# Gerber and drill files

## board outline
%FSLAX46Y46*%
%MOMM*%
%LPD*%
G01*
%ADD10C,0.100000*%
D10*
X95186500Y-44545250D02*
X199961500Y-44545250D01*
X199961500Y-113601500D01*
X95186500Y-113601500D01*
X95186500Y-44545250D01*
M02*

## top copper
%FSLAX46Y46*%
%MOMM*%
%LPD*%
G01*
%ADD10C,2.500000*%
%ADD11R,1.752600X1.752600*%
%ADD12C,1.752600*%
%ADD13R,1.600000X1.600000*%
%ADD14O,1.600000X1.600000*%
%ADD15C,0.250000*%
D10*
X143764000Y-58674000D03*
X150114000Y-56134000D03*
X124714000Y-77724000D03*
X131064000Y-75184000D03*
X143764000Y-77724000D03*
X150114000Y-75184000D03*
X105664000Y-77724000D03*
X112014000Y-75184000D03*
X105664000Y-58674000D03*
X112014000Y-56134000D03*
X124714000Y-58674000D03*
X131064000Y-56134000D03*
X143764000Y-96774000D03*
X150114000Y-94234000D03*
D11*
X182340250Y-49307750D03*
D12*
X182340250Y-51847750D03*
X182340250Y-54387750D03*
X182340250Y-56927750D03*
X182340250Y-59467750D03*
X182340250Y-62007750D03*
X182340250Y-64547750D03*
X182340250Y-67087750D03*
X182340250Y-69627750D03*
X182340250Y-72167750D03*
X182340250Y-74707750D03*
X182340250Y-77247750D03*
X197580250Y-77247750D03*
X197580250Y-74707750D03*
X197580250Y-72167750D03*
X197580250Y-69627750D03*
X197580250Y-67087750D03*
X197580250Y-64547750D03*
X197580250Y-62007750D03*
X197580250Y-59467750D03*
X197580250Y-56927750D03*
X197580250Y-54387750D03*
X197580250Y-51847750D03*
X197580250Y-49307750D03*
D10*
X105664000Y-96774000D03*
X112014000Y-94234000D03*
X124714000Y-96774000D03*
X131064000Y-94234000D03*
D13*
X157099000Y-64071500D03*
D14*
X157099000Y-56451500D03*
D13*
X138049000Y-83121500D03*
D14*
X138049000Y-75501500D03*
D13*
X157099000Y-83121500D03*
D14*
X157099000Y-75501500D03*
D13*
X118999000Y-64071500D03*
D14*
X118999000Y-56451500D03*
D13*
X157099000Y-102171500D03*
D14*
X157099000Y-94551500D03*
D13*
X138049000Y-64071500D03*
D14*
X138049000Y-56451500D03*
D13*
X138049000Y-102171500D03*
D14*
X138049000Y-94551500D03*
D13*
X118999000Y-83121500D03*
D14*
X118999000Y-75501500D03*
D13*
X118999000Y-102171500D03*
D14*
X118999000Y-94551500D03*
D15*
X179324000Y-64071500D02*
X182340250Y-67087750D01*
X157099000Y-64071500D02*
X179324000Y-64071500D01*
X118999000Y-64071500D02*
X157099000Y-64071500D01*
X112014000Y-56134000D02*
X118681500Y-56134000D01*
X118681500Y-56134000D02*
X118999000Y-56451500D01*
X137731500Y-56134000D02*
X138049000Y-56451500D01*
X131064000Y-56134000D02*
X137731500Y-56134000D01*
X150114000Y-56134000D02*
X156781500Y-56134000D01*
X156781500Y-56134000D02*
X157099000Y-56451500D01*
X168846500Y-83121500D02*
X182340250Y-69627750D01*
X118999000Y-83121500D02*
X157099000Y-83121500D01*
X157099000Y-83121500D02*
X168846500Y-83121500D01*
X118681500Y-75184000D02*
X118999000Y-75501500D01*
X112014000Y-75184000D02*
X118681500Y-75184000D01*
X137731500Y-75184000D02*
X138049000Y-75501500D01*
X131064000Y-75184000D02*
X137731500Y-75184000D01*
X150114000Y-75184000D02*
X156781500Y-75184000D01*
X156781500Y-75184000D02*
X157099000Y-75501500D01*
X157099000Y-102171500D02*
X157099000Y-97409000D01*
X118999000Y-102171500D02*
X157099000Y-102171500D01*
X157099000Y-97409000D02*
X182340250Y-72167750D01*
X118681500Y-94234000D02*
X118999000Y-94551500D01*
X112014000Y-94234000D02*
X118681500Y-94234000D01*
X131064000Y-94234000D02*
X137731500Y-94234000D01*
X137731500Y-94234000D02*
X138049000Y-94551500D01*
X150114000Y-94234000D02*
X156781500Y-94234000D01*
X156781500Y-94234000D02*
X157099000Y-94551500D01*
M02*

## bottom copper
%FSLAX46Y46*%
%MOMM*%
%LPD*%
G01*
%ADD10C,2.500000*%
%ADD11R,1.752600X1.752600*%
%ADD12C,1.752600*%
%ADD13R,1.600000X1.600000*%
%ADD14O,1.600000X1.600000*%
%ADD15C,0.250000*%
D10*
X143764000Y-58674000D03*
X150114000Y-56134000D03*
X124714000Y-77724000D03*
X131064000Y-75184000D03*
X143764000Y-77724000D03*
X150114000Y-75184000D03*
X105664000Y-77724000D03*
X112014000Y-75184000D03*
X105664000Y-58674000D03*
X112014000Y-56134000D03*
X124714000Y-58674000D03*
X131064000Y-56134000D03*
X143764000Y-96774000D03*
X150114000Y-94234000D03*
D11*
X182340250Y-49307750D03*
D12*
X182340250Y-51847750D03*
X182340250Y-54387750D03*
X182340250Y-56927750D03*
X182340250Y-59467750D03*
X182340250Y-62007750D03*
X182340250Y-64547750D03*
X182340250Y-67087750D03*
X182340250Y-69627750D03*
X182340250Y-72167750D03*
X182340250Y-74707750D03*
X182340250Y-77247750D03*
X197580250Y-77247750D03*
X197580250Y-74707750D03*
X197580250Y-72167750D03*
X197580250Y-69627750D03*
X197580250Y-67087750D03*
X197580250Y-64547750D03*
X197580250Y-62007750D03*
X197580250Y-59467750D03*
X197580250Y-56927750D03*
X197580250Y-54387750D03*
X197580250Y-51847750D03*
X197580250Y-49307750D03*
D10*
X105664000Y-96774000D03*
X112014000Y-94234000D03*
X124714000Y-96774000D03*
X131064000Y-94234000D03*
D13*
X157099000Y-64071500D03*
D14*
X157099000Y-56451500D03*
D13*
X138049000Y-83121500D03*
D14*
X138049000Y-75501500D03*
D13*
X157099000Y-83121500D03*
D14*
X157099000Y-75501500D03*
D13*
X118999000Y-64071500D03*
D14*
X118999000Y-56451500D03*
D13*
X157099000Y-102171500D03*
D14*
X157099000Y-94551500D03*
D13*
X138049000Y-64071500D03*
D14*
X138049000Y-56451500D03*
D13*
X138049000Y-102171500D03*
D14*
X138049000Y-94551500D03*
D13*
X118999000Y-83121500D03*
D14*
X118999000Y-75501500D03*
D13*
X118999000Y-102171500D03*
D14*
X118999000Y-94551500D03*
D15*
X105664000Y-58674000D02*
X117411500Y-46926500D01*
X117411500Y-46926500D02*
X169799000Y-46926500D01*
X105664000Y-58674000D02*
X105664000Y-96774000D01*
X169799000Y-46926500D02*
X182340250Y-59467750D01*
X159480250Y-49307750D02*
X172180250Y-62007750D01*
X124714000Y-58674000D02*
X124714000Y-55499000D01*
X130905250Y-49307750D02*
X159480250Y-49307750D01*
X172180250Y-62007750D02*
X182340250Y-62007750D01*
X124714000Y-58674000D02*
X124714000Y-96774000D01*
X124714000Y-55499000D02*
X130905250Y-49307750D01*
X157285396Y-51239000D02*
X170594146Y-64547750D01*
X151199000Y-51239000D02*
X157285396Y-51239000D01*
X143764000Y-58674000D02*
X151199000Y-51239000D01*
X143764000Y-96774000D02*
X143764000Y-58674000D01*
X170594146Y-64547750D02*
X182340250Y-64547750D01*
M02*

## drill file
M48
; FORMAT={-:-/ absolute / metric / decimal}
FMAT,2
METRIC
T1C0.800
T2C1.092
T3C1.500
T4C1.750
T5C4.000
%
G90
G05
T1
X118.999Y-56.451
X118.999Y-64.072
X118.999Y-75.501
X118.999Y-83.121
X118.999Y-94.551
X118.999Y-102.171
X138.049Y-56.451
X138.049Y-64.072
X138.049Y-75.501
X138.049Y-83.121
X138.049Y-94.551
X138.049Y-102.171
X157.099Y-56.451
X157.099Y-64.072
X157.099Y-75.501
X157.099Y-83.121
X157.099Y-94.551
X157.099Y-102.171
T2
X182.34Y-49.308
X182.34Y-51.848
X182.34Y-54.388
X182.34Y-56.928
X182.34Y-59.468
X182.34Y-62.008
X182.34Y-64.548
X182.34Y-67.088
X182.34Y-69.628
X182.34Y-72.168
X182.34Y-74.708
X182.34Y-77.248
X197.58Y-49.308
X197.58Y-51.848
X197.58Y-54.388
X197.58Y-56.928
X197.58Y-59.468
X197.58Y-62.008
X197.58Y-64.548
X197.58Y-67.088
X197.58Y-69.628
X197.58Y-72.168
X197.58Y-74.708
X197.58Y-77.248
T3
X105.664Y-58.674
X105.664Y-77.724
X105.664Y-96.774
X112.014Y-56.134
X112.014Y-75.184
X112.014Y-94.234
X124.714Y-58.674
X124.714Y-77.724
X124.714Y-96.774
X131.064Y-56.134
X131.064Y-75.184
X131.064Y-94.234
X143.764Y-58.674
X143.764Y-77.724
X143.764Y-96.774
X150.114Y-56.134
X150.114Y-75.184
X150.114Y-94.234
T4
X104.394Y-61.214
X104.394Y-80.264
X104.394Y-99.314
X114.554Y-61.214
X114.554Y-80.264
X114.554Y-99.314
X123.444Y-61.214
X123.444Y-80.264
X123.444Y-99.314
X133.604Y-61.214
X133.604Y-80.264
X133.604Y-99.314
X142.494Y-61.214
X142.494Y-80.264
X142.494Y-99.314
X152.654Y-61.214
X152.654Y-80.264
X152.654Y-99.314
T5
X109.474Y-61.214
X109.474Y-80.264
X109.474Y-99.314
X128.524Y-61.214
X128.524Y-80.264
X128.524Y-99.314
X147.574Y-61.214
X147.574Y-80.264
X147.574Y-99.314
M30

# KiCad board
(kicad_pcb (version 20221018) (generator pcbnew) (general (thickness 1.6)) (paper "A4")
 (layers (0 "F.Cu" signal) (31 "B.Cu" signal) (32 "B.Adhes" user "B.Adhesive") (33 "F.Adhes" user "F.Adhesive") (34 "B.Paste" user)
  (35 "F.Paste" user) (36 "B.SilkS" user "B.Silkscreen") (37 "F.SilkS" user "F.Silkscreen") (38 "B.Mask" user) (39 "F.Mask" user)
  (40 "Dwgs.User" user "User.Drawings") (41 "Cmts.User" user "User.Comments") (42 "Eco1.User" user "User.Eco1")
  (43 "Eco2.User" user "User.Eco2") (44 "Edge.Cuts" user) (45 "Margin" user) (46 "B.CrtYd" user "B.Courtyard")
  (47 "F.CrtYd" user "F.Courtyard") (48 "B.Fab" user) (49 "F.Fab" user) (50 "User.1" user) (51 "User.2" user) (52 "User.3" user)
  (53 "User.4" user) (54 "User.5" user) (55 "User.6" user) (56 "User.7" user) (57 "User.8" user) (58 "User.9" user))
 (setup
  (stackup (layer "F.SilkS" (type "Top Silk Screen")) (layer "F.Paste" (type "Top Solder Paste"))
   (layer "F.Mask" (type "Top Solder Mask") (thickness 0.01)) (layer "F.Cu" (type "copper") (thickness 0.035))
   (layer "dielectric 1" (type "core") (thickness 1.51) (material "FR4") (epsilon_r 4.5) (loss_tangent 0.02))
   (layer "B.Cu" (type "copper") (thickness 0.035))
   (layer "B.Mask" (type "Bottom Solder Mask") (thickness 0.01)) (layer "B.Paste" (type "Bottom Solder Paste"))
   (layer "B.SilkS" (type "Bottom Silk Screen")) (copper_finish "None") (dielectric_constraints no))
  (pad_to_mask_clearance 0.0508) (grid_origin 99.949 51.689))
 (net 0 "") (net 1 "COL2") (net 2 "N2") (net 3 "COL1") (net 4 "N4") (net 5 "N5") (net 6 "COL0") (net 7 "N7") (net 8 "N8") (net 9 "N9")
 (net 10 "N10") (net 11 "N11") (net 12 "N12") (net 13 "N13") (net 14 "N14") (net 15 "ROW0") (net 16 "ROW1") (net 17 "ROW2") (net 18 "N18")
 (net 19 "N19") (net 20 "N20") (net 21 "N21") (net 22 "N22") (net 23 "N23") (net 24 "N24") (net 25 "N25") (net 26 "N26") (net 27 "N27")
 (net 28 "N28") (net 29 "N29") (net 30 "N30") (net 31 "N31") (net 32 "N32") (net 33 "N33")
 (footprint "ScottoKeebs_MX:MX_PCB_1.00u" (layer "F.Cu") (at 147.574 61.214)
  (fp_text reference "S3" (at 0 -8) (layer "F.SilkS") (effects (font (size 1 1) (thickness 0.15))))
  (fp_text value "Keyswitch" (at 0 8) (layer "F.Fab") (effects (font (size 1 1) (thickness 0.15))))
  (pad "" np_thru_hole circle (at -5.08 0) (size 1.75 1.75) (drill 1.75) (layers "*.Cu" "*.Mask"))
  (pad "" np_thru_hole circle (at 0 0) (size 4 4) (drill 4) (layers "*.Cu" "*.Mask"))
  (pad "" np_thru_hole circle (at 5.08 0) (size 1.75 1.75) (drill 1.75) (layers "*.Cu" "*.Mask"))
  (pad "1" thru_hole circle (at -3.81 -2.54) (size 2.5 2.5) (drill 1.5) (layers "*.Cu" "*.Mask") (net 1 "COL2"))
  (pad "2" thru_hole circle (at 2.54 -5.08) (size 2.5 2.5) (drill 1.5) (layers "*.Cu" "*.Mask") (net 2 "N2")))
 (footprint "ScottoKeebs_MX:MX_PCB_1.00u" (layer "F.Cu") (at 128.524 80.264)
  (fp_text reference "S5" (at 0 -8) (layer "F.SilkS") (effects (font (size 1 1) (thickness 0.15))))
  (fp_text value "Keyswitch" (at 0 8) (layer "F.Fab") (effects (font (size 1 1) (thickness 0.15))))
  (pad "" np_thru_hole circle (at -5.08 0) (size 1.75 1.75) (drill 1.75) (layers "*.Cu" "*.Mask"))
  (pad "" np_thru_hole circle (at 0 0) (size 4 4) (drill 4) (layers "*.Cu" "*.Mask"))
  (pad "" np_thru_hole circle (at 5.08 0) (size 1.75 1.75) (drill 1.75) (layers "*.Cu" "*.Mask"))
  (pad "1" thru_hole circle (at -3.81 -2.54) (size 2.5 2.5) (drill 1.5) (layers "*.Cu" "*.Mask") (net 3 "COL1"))
  (pad "2" thru_hole circle (at 2.54 -5.08) (size 2.5 2.5) (drill 1.5) (layers "*.Cu" "*.Mask") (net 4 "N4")))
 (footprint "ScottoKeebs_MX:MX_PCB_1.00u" (layer "F.Cu") (at 147.574 80.264)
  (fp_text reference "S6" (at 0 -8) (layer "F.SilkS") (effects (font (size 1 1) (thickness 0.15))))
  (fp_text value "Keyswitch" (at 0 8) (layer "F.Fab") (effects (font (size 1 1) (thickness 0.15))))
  (pad "" np_thru_hole circle (at -5.08 0) (size 1.75 1.75) (drill 1.75) (layers "*.Cu" "*.Mask"))
  (pad "" np_thru_hole circle (at 0 0) (size 4 4) (drill 4) (layers "*.Cu" "*.Mask"))
  (pad "" np_thru_hole circle (at 5.08 0) (size 1.75 1.75) (drill 1.75) (layers "*.Cu" "*.Mask"))
  (pad "1" thru_hole circle (at -3.81 -2.54) (size 2.5 2.5) (drill 1.5) (layers "*.Cu" "*.Mask") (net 1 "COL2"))
  (pad "2" thru_hole circle (at 2.54 -5.08) (size 2.5 2.5) (drill 1.5) (layers "*.Cu" "*.Mask") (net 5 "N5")))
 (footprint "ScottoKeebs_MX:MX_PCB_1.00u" (layer "F.Cu") (at 109.474 80.264)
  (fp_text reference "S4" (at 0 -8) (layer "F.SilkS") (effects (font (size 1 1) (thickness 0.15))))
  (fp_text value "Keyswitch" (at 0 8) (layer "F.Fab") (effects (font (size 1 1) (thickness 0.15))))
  (pad "" np_thru_hole circle (at -5.08 0) (size 1.75 1.75) (drill 1.75) (layers "*.Cu" "*.Mask"))
  (pad "" np_thru_hole circle (at 0 0) (size 4 4) (drill 4) (layers "*.Cu" "*.Mask"))
  (pad "" np_thru_hole circle (at 5.08 0) (size 1.75 1.75) (drill 1.75) (layers "*.Cu" "*.Mask"))
  (pad "1" thru_hole circle (at -3.81 -2.54) (size 2.5 2.5) (drill 1.5) (layers "*.Cu" "*.Mask") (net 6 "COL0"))
  (pad "2" thru_hole circle (at 2.54 -5.08) (size 2.5 2.5) (drill 1.5) (layers "*.Cu" "*.Mask") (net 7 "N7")))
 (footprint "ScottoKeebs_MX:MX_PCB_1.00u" (layer "F.Cu") (at 109.474 61.214)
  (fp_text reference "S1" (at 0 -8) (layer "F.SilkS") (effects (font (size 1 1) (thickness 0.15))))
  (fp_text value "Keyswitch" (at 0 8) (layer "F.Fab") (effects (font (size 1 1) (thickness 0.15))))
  (pad "" np_thru_hole circle (at -5.08 0) (size 1.75 1.75) (drill 1.75) (layers "*.Cu" "*.Mask"))
  (pad "" np_thru_hole circle (at 0 0) (size 4 4) (drill 4) (layers "*.Cu" "*.Mask"))
  (pad "" np_thru_hole circle (at 5.08 0) (size 1.75 1.75) (drill 1.75) (layers "*.Cu" "*.Mask"))
  (pad "1" thru_hole circle (at -3.81 -2.54) (size 2.5 2.5) (drill 1.5) (layers "*.Cu" "*.Mask") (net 6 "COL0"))
  (pad "2" thru_hole circle (at 2.54 -5.08) (size 2.5 2.5) (drill 1.5) (layers "*.Cu" "*.Mask") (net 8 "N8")))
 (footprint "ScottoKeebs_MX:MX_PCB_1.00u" (layer "F.Cu") (at 128.524 61.214)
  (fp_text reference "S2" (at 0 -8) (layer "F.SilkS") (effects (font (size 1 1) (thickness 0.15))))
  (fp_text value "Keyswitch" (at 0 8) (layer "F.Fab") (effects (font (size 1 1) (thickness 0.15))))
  (pad "" np_thru_hole circle (at -5.08 0) (size 1.75 1.75) (drill 1.75) (layers "*.Cu" "*.Mask"))
  (pad "" np_thru_hole circle (at 0 0) (size 4 4) (drill 4) (layers "*.Cu" "*.Mask"))
  (pad "" np_thru_hole circle (at 5.08 0) (size 1.75 1.75) (drill 1.75) (layers "*.Cu" "*.Mask"))
  (pad "1" thru_hole circle (at -3.81 -2.54) (size 2.5 2.5) (drill 1.5) (layers "*.Cu" "*.Mask") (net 3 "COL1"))
  (pad "2" thru_hole circle (at 2.54 -5.08) (size 2.5 2.5) (drill 1.5) (layers "*.Cu" "*.Mask") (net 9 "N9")))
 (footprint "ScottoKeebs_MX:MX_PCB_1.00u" (layer "F.Cu") (at 147.574 99.314)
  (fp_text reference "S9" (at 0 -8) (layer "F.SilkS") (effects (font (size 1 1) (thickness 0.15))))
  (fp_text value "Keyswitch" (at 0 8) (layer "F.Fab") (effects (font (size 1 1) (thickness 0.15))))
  (pad "" np_thru_hole circle (at -5.08 0) (size 1.75 1.75) (drill 1.75) (layers "*.Cu" "*.Mask"))
  (pad "" np_thru_hole circle (at 0 0) (size 4 4) (drill 4) (layers "*.Cu" "*.Mask"))
  (pad "" np_thru_hole circle (at 5.08 0) (size 1.75 1.75) (drill 1.75) (layers "*.Cu" "*.Mask"))
  (pad "1" thru_hole circle (at -3.81 -2.54) (size 2.5 2.5) (drill 1.5) (layers "*.Cu" "*.Mask") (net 1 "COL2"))
  (pad "2" thru_hole circle (at 2.54 -5.08) (size 2.5 2.5) (drill 1.5) (layers "*.Cu" "*.Mask") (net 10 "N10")))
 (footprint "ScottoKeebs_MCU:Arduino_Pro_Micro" (layer "F.Cu") (at 189.96025 63.27775)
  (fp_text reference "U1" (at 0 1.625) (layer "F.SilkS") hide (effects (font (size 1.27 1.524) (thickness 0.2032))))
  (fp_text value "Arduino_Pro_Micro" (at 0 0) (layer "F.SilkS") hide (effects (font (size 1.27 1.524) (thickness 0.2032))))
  (pad "1" thru_hole rect (at -7.62 -13.97 270) (size 1.7526 1.7526) (drill 1.0922) (layers "*.Cu" "*.Mask") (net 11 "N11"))
  (pad "2" thru_hole circle (at -7.62 -11.43 270) (size 1.7526 1.7526) (drill 1.0922) (layers "*.Cu" "*.Mask") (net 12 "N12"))
  (pad "3" thru_hole circle (at -7.62 -8.89 270) (size 1.7526 1.7526) (drill 1.0922) (layers "*.Cu" "*.Mask") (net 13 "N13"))
  (pad "4" thru_hole circle (at -7.62 -6.35 270) (size 1.7526 1.7526) (drill 1.0922) (layers "*.Cu" "*.Mask") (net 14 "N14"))
  (pad "5" thru_hole circle (at -7.62 -3.81 270) (size 1.7526 1.7526) (drill 1.0922) (layers "*.Cu" "*.Mask") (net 6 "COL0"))
  (pad "6" thru_hole circle (at -7.62 -1.27 270) (size 1.7526 1.7526) (drill 1.0922) (layers "*.Cu" "*.Mask") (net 3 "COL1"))
  (pad "7" thru_hole circle (at -7.62 1.27 270) (size 1.7526 1.7526) (drill 1.0922) (layers "*.Cu" "*.Mask") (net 1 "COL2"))
  (pad "8" thru_hole circle (at -7.62 3.81 270) (size 1.7526 1.7526) (drill 1.0922) (layers "*.Cu" "*.Mask") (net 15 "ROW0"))
  (pad "9" thru_hole circle (at -7.62 6.35 270) (size 1.7526 1.7526) (drill 1.0922) (layers "*.Cu" "*.Mask") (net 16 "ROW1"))
  (pad "10" thru_hole circle (at -7.62 8.89 270) (size 1.7526 1.7526) (drill 1.0922) (layers "*.Cu" "*.Mask") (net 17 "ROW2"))
  (pad "11" thru_hole circle (at -7.62 11.43 270) (size 1.7526 1.7526) (drill 1.0922) (layers "*.Cu" "*.Mask") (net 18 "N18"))
  (pad "12" thru_hole circle (at -7.62 13.97 270) (size 1.7526 1.7526) (drill 1.0922) (layers "*.Cu" "*.Mask") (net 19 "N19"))
  (pad "13" thru_hole circle (at 7.62 13.97 270) (size 1.7526 1.7526) (drill 1.0922) (layers "*.Cu" "*.Mask") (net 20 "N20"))
  (pad "14" thru_hole circle (at 7.62 11.43 270) (size 1.7526 1.7526) (drill 1.0922) (layers "*.Cu" "*.Mask") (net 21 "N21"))
  (pad "15" thru_hole circle (at 7.62 8.89 270) (size 1.7526 1.7526) (drill 1.0922) (layers "*.Cu" "*.Mask") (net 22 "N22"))
  (pad "16" thru_hole circle (at 7.62 6.35 270) (size 1.7526 1.7526) (drill 1.0922) (layers "*.Cu" "*.Mask") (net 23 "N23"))
  (pad "17" thru_hole circle (at 7.62 3.81 270) (size 1.7526 1.7526) (drill 1.0922) (layers "*.Cu" "*.Mask") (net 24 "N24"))
  (pad "18" thru_hole circle (at 7.62 1.27 270) (size 1.7526 1.7526) (drill 1.0922) (layers "*.Cu" "*.Mask") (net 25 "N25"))
  (pad "19" thru_hole circle (at 7.62 -1.27 270) (size 1.7526 1.7526) (drill 1.0922) (layers "*.Cu" "*.Mask") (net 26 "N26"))
  (pad "20" thru_hole circle (at 7.62 -3.81 270) (size 1.7526 1.7526) (drill 1.0922) (layers "*.Cu" "*.Mask") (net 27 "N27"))
  (pad "21" thru_hole circle (at 7.62 -6.35 270) (size 1.7526 1.7526) (drill 1.0922) (layers "*.Cu" "*.Mask") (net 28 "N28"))
  (pad "22" thru_hole circle (at 7.62 -8.89 270) (size 1.7526 1.7526) (drill 1.0922) (layers "*.Cu" "*.Mask") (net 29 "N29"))
  (pad "23" thru_hole circle (at 7.62 -11.43 270) (size 1.7526 1.7526) (drill 1.0922) (layers "*.Cu" "*.Mask") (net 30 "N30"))
  (pad "24" thru_hole circle (at 7.62 -13.97 270) (size 1.7526 1.7526) (drill 1.0922) (layers "*.Cu" "*.Mask") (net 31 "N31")))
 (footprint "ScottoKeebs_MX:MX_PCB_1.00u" (layer "F.Cu") (at 109.474 99.314)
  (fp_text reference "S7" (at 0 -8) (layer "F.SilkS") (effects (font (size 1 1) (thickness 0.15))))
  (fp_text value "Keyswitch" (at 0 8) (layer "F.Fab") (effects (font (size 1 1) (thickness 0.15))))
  (pad "" np_thru_hole circle (at -5.08 0) (size 1.75 1.75) (drill 1.75) (layers "*.Cu" "*.Mask"))
  (pad "" np_thru_hole circle (at 0 0) (size 4 4) (drill 4) (layers "*.Cu" "*.Mask"))
  (pad "" np_thru_hole circle (at 5.08 0) (size 1.75 1.75) (drill 1.75) (layers "*.Cu" "*.Mask"))
  (pad "1" thru_hole circle (at -3.81 -2.54) (size 2.5 2.5) (drill 1.5) (layers "*.Cu" "*.Mask") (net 6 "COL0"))
  (pad "2" thru_hole circle (at 2.54 -5.08) (size 2.5 2.5) (drill 1.5) (layers "*.Cu" "*.Mask") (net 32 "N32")))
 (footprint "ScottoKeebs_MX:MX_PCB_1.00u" (layer "F.Cu") (at 128.524 99.314)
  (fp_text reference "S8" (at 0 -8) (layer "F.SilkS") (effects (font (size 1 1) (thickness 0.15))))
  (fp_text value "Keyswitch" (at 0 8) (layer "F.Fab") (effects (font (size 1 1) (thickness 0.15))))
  (pad "" np_thru_hole circle (at -5.08 0) (size 1.75 1.75) (drill 1.75) (layers "*.Cu" "*.Mask"))
  (pad "" np_thru_hole circle (at 0 0) (size 4 4) (drill 4) (layers "*.Cu" "*.Mask"))
  (pad "" np_thru_hole circle (at 5.08 0) (size 1.75 1.75) (drill 1.75) (layers "*.Cu" "*.Mask"))
  (pad "1" thru_hole circle (at -3.81 -2.54) (size 2.5 2.5) (drill 1.5) (layers "*.Cu" "*.Mask") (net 3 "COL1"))
  (pad "2" thru_hole circle (at 2.54 -5.08) (size 2.5 2.5) (drill 1.5) (layers "*.Cu" "*.Mask") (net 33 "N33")))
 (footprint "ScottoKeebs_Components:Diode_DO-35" (layer "B.Cu") (at 157.099 64.0715 90)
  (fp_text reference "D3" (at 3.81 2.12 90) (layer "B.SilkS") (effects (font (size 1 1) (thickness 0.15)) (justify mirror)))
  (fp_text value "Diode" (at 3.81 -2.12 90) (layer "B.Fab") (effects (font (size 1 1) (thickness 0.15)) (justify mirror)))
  (pad "1" thru_hole rect (at 0 0 90) (size 1.6 1.6) (drill 0.8) (layers "*.Cu" "*.Mask") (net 15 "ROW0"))
  (pad "2" thru_hole oval (at 7.62 0 90) (size 1.6 1.6) (drill 0.8) (layers "*.Cu" "*.Mask") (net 2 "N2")))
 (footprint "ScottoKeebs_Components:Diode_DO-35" (layer "B.Cu") (at 138.049 83.1215 90)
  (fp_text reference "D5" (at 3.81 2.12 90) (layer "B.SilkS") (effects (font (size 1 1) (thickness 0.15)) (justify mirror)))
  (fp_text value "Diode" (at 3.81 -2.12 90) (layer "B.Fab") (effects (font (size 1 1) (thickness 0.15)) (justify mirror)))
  (pad "1" thru_hole rect (at 0 0 90) (size 1.6 1.6) (drill 0.8) (layers "*.Cu" "*.Mask") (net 16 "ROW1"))
  (pad "2" thru_hole oval (at 7.62 0 90) (size 1.6 1.6) (drill 0.8) (layers "*.Cu" "*.Mask") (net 4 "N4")))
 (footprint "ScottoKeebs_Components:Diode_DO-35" (layer "B.Cu") (at 157.099 83.1215 90)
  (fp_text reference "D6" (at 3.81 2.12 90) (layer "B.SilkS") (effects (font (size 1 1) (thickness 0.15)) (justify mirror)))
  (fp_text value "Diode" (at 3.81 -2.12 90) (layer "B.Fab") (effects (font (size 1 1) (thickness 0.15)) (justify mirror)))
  (pad "1" thru_hole rect (at 0 0 90) (size 1.6 1.6) (drill 0.8) (layers "*.Cu" "*.Mask") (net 16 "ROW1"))
  (pad "2" thru_hole oval (at 7.62 0 90) (size 1.6 1.6) (drill 0.8) (layers "*.Cu" "*.Mask") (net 5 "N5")))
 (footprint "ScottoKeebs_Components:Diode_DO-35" (layer "B.Cu") (at 118.999 64.0715 90)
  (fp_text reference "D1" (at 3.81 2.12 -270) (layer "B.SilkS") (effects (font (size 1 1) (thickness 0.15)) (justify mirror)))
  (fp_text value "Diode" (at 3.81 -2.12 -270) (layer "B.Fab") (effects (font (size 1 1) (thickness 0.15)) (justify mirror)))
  (pad "1" thru_hole rect (at 0 0 90) (size 1.6 1.6) (drill 0.8) (layers "*.Cu" "*.Mask") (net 15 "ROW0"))
  (pad "2" thru_hole oval (at 7.62 0 90) (size 1.6 1.6) (drill 0.8) (layers "*.Cu" "*.Mask") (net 8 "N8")))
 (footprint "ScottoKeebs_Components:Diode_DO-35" (layer "B.Cu") (at 157.099 102.1715 90)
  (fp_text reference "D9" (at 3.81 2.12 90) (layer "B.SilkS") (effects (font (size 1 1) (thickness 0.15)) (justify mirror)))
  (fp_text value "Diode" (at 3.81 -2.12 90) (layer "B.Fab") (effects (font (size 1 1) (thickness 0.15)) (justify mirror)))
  (pad "1" thru_hole rect (at 0 0 90) (size 1.6 1.6) (drill 0.8) (layers "*.Cu" "*.Mask") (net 17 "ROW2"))
  (pad "2" thru_hole oval (at 7.62 0 90) (size 1.6 1.6) (drill 0.8) (layers "*.Cu" "*.Mask") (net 10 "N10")))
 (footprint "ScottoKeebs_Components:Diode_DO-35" (layer "B.Cu") (at 138.049 64.0715 90)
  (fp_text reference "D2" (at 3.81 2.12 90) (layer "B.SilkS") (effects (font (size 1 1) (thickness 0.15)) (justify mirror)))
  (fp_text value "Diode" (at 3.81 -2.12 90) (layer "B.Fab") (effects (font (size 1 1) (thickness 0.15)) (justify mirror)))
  (pad "1" thru_hole rect (at 0 0 90) (size 1.6 1.6) (drill 0.8) (layers "*.Cu" "*.Mask") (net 15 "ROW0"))
  (pad "2" thru_hole oval (at 7.62 0 90) (size 1.6 1.6) (drill 0.8) (layers "*.Cu" "*.Mask") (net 9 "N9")))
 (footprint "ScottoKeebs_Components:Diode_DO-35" (layer "B.Cu") (at 138.049 102.1715 90)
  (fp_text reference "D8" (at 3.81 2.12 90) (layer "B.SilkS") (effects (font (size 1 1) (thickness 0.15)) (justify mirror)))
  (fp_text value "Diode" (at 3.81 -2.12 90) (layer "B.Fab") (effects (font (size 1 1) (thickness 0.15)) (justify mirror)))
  (pad "1" thru_hole rect (at 0 0 90) (size 1.6 1.6) (drill 0.8) (layers "*.Cu" "*.Mask") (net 17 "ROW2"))
  (pad "2" thru_hole oval (at 7.62 0 90) (size 1.6 1.6) (drill 0.8) (layers "*.Cu" "*.Mask") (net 33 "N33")))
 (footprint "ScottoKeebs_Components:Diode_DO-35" (layer "B.Cu") (at 118.999 83.1215 90)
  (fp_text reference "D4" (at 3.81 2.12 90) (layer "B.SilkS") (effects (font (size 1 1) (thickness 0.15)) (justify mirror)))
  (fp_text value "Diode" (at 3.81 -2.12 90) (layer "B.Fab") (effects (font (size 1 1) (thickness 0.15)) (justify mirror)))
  (pad "1" thru_hole rect (at 0 0 90) (size 1.6 1.6) (drill 0.8) (layers "*.Cu" "*.Mask") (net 16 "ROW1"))
  (pad "2" thru_hole oval (at 7.62 0 90) (size 1.6 1.6) (drill 0.8) (layers "*.Cu" "*.Mask") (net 7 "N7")))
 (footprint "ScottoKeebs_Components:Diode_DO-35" (layer "B.Cu") (at 118.999 102.1715 90)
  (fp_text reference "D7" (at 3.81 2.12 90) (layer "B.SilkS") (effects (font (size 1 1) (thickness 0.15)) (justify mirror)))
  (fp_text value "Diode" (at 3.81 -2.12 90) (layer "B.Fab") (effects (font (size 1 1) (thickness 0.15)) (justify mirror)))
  (pad "1" thru_hole rect (at 0 0 90) (size 1.6 1.6) (drill 0.8) (layers "*.Cu" "*.Mask") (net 17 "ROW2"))
  (pad "2" thru_hole oval (at 7.62 0 90) (size 1.6 1.6) (drill 0.8) (layers "*.Cu" "*.Mask") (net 32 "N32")))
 (gr_rect (start 95.1865 44.54525) (end 199.9615 113.6015) (stroke (width 0.1) (type default)) (fill none) (layer "Edge.Cuts"))
 (segment (start 179.324 64.0715) (end 182.34025 67.08775) (width 0.25) (layer "F.Cu") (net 15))
 (segment (start 157.099 64.0715) (end 179.324 64.0715) (width 0.25) (layer "F.Cu") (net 15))
 (segment (start 118.999 64.0715) (end 157.099 64.0715) (width 0.25) (layer "F.Cu") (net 15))
 (segment (start 112.014 56.134) (end 118.6815 56.134) (width 0.25) (layer "F.Cu") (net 8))
 (segment (start 118.6815 56.134) (end 118.999 56.4515) (width 0.25) (layer "F.Cu") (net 8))
 (segment (start 137.7315 56.134) (end 138.049 56.4515) (width 0.25) (layer "F.Cu") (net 9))
 (segment (start 131.064 56.134) (end 137.7315 56.134) (width 0.25) (layer "F.Cu") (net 9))
 (segment (start 150.114 56.134) (end 156.7815 56.134) (width 0.25) (layer "F.Cu") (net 2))
 (segment (start 156.7815 56.134) (end 157.099 56.4515) (width 0.25) (layer "F.Cu") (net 2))
 (segment (start 168.8465 83.1215) (end 182.34025 69.62775) (width 0.25) (layer "F.Cu") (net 16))
 (segment (start 118.999 83.1215) (end 157.099 83.1215) (width 0.25) (layer "F.Cu") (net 16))
 (segment (start 157.099 83.1215) (end 168.8465 83.1215) (width 0.25) (layer "F.Cu") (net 16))
 (segment (start 118.6815 75.184) (end 118.999 75.5015) (width 0.25) (layer "F.Cu") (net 7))
 (segment (start 112.014 75.184) (end 118.6815 75.184) (width 0.25) (layer "F.Cu") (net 7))
 (segment (start 137.7315 75.184) (end 138.049 75.5015) (width 0.25) (layer "F.Cu") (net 4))
 (segment (start 131.064 75.184) (end 137.7315 75.184) (width 0.25) (layer "F.Cu") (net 4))
 (segment (start 150.114 75.184) (end 156.7815 75.184) (width 0.25) (layer "F.Cu") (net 5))
 (segment (start 156.7815 75.184) (end 157.099 75.5015) (width 0.25) (layer "F.Cu") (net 5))
 (segment (start 157.099 102.1715) (end 157.099 97.409) (width 0.25) (layer "F.Cu") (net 17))
 (segment (start 118.999 102.1715) (end 157.099 102.1715) (width 0.25) (layer "F.Cu") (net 17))
 (segment (start 157.099 97.409) (end 182.34025 72.16775) (width 0.25) (layer "F.Cu") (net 17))
 (segment (start 118.6815 94.234) (end 118.999 94.5515) (width 0.25) (layer "F.Cu") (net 32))
 (segment (start 112.014 94.234) (end 118.6815 94.234) (width 0.25) (layer "F.Cu") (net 32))
 (segment (start 131.064 94.234) (end 137.7315 94.234) (width 0.25) (layer "F.Cu") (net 33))
 (segment (start 137.7315 94.234) (end 138.049 94.5515) (width 0.25) (layer "F.Cu") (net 33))
 (segment (start 150.114 94.234) (end 156.7815 94.234) (width 0.25) (layer "F.Cu") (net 10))
 (segment (start 156.7815 94.234) (end 157.099 94.5515) (width 0.25) (layer "F.Cu") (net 10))
 (segment (start 105.664 58.674) (end 117.4115 46.9265) (width 0.25) (layer "B.Cu") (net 6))
 (segment (start 117.4115 46.9265) (end 169.799 46.9265) (width 0.25) (layer "B.Cu") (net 6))
 (segment (start 105.664 58.674) (end 105.664 96.774) (width 0.25) (layer "B.Cu") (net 6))
 (segment (start 169.799 46.9265) (end 182.34025 59.46775) (width 0.25) (layer "B.Cu") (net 6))
 (segment (start 159.48025 49.30775) (end 172.18025 62.00775) (width 0.25) (layer "B.Cu") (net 3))
 (segment (start 124.714 58.674) (end 124.714 55.499) (width 0.25) (layer "B.Cu") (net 3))
 (segment (start 130.90525 49.30775) (end 159.48025 49.30775) (width 0.25) (layer "B.Cu") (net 3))
 (segment (start 172.18025 62.00775) (end 182.34025 62.00775) (width 0.25) (layer "B.Cu") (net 3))
 (segment (start 124.714 58.674) (end 124.714 96.774) (width 0.25) (layer "B.Cu") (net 3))
 (segment (start 124.714 55.499) (end 130.90525 49.30775) (width 0.25) (layer "B.Cu") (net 3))
 (segment (start 157.285396 51.239) (end 170.594146 64.54775) (width 0.25) (layer "B.Cu") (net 1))
 (segment (start 151.199 51.239) (end 157.285396 51.239) (width 0.25) (layer "B.Cu") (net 1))
 (segment (start 143.764 58.674) (end 151.199 51.239) (width 0.25) (layer "B.Cu") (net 1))
 (segment (start 143.764 96.774) (end 143.764 58.674) (width 0.25) (layer "B.Cu") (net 1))
 (segment (start 170.594146 64.54775) (end 182.34025 64.54775) (width 0.25) (layer "B.Cu") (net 1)))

